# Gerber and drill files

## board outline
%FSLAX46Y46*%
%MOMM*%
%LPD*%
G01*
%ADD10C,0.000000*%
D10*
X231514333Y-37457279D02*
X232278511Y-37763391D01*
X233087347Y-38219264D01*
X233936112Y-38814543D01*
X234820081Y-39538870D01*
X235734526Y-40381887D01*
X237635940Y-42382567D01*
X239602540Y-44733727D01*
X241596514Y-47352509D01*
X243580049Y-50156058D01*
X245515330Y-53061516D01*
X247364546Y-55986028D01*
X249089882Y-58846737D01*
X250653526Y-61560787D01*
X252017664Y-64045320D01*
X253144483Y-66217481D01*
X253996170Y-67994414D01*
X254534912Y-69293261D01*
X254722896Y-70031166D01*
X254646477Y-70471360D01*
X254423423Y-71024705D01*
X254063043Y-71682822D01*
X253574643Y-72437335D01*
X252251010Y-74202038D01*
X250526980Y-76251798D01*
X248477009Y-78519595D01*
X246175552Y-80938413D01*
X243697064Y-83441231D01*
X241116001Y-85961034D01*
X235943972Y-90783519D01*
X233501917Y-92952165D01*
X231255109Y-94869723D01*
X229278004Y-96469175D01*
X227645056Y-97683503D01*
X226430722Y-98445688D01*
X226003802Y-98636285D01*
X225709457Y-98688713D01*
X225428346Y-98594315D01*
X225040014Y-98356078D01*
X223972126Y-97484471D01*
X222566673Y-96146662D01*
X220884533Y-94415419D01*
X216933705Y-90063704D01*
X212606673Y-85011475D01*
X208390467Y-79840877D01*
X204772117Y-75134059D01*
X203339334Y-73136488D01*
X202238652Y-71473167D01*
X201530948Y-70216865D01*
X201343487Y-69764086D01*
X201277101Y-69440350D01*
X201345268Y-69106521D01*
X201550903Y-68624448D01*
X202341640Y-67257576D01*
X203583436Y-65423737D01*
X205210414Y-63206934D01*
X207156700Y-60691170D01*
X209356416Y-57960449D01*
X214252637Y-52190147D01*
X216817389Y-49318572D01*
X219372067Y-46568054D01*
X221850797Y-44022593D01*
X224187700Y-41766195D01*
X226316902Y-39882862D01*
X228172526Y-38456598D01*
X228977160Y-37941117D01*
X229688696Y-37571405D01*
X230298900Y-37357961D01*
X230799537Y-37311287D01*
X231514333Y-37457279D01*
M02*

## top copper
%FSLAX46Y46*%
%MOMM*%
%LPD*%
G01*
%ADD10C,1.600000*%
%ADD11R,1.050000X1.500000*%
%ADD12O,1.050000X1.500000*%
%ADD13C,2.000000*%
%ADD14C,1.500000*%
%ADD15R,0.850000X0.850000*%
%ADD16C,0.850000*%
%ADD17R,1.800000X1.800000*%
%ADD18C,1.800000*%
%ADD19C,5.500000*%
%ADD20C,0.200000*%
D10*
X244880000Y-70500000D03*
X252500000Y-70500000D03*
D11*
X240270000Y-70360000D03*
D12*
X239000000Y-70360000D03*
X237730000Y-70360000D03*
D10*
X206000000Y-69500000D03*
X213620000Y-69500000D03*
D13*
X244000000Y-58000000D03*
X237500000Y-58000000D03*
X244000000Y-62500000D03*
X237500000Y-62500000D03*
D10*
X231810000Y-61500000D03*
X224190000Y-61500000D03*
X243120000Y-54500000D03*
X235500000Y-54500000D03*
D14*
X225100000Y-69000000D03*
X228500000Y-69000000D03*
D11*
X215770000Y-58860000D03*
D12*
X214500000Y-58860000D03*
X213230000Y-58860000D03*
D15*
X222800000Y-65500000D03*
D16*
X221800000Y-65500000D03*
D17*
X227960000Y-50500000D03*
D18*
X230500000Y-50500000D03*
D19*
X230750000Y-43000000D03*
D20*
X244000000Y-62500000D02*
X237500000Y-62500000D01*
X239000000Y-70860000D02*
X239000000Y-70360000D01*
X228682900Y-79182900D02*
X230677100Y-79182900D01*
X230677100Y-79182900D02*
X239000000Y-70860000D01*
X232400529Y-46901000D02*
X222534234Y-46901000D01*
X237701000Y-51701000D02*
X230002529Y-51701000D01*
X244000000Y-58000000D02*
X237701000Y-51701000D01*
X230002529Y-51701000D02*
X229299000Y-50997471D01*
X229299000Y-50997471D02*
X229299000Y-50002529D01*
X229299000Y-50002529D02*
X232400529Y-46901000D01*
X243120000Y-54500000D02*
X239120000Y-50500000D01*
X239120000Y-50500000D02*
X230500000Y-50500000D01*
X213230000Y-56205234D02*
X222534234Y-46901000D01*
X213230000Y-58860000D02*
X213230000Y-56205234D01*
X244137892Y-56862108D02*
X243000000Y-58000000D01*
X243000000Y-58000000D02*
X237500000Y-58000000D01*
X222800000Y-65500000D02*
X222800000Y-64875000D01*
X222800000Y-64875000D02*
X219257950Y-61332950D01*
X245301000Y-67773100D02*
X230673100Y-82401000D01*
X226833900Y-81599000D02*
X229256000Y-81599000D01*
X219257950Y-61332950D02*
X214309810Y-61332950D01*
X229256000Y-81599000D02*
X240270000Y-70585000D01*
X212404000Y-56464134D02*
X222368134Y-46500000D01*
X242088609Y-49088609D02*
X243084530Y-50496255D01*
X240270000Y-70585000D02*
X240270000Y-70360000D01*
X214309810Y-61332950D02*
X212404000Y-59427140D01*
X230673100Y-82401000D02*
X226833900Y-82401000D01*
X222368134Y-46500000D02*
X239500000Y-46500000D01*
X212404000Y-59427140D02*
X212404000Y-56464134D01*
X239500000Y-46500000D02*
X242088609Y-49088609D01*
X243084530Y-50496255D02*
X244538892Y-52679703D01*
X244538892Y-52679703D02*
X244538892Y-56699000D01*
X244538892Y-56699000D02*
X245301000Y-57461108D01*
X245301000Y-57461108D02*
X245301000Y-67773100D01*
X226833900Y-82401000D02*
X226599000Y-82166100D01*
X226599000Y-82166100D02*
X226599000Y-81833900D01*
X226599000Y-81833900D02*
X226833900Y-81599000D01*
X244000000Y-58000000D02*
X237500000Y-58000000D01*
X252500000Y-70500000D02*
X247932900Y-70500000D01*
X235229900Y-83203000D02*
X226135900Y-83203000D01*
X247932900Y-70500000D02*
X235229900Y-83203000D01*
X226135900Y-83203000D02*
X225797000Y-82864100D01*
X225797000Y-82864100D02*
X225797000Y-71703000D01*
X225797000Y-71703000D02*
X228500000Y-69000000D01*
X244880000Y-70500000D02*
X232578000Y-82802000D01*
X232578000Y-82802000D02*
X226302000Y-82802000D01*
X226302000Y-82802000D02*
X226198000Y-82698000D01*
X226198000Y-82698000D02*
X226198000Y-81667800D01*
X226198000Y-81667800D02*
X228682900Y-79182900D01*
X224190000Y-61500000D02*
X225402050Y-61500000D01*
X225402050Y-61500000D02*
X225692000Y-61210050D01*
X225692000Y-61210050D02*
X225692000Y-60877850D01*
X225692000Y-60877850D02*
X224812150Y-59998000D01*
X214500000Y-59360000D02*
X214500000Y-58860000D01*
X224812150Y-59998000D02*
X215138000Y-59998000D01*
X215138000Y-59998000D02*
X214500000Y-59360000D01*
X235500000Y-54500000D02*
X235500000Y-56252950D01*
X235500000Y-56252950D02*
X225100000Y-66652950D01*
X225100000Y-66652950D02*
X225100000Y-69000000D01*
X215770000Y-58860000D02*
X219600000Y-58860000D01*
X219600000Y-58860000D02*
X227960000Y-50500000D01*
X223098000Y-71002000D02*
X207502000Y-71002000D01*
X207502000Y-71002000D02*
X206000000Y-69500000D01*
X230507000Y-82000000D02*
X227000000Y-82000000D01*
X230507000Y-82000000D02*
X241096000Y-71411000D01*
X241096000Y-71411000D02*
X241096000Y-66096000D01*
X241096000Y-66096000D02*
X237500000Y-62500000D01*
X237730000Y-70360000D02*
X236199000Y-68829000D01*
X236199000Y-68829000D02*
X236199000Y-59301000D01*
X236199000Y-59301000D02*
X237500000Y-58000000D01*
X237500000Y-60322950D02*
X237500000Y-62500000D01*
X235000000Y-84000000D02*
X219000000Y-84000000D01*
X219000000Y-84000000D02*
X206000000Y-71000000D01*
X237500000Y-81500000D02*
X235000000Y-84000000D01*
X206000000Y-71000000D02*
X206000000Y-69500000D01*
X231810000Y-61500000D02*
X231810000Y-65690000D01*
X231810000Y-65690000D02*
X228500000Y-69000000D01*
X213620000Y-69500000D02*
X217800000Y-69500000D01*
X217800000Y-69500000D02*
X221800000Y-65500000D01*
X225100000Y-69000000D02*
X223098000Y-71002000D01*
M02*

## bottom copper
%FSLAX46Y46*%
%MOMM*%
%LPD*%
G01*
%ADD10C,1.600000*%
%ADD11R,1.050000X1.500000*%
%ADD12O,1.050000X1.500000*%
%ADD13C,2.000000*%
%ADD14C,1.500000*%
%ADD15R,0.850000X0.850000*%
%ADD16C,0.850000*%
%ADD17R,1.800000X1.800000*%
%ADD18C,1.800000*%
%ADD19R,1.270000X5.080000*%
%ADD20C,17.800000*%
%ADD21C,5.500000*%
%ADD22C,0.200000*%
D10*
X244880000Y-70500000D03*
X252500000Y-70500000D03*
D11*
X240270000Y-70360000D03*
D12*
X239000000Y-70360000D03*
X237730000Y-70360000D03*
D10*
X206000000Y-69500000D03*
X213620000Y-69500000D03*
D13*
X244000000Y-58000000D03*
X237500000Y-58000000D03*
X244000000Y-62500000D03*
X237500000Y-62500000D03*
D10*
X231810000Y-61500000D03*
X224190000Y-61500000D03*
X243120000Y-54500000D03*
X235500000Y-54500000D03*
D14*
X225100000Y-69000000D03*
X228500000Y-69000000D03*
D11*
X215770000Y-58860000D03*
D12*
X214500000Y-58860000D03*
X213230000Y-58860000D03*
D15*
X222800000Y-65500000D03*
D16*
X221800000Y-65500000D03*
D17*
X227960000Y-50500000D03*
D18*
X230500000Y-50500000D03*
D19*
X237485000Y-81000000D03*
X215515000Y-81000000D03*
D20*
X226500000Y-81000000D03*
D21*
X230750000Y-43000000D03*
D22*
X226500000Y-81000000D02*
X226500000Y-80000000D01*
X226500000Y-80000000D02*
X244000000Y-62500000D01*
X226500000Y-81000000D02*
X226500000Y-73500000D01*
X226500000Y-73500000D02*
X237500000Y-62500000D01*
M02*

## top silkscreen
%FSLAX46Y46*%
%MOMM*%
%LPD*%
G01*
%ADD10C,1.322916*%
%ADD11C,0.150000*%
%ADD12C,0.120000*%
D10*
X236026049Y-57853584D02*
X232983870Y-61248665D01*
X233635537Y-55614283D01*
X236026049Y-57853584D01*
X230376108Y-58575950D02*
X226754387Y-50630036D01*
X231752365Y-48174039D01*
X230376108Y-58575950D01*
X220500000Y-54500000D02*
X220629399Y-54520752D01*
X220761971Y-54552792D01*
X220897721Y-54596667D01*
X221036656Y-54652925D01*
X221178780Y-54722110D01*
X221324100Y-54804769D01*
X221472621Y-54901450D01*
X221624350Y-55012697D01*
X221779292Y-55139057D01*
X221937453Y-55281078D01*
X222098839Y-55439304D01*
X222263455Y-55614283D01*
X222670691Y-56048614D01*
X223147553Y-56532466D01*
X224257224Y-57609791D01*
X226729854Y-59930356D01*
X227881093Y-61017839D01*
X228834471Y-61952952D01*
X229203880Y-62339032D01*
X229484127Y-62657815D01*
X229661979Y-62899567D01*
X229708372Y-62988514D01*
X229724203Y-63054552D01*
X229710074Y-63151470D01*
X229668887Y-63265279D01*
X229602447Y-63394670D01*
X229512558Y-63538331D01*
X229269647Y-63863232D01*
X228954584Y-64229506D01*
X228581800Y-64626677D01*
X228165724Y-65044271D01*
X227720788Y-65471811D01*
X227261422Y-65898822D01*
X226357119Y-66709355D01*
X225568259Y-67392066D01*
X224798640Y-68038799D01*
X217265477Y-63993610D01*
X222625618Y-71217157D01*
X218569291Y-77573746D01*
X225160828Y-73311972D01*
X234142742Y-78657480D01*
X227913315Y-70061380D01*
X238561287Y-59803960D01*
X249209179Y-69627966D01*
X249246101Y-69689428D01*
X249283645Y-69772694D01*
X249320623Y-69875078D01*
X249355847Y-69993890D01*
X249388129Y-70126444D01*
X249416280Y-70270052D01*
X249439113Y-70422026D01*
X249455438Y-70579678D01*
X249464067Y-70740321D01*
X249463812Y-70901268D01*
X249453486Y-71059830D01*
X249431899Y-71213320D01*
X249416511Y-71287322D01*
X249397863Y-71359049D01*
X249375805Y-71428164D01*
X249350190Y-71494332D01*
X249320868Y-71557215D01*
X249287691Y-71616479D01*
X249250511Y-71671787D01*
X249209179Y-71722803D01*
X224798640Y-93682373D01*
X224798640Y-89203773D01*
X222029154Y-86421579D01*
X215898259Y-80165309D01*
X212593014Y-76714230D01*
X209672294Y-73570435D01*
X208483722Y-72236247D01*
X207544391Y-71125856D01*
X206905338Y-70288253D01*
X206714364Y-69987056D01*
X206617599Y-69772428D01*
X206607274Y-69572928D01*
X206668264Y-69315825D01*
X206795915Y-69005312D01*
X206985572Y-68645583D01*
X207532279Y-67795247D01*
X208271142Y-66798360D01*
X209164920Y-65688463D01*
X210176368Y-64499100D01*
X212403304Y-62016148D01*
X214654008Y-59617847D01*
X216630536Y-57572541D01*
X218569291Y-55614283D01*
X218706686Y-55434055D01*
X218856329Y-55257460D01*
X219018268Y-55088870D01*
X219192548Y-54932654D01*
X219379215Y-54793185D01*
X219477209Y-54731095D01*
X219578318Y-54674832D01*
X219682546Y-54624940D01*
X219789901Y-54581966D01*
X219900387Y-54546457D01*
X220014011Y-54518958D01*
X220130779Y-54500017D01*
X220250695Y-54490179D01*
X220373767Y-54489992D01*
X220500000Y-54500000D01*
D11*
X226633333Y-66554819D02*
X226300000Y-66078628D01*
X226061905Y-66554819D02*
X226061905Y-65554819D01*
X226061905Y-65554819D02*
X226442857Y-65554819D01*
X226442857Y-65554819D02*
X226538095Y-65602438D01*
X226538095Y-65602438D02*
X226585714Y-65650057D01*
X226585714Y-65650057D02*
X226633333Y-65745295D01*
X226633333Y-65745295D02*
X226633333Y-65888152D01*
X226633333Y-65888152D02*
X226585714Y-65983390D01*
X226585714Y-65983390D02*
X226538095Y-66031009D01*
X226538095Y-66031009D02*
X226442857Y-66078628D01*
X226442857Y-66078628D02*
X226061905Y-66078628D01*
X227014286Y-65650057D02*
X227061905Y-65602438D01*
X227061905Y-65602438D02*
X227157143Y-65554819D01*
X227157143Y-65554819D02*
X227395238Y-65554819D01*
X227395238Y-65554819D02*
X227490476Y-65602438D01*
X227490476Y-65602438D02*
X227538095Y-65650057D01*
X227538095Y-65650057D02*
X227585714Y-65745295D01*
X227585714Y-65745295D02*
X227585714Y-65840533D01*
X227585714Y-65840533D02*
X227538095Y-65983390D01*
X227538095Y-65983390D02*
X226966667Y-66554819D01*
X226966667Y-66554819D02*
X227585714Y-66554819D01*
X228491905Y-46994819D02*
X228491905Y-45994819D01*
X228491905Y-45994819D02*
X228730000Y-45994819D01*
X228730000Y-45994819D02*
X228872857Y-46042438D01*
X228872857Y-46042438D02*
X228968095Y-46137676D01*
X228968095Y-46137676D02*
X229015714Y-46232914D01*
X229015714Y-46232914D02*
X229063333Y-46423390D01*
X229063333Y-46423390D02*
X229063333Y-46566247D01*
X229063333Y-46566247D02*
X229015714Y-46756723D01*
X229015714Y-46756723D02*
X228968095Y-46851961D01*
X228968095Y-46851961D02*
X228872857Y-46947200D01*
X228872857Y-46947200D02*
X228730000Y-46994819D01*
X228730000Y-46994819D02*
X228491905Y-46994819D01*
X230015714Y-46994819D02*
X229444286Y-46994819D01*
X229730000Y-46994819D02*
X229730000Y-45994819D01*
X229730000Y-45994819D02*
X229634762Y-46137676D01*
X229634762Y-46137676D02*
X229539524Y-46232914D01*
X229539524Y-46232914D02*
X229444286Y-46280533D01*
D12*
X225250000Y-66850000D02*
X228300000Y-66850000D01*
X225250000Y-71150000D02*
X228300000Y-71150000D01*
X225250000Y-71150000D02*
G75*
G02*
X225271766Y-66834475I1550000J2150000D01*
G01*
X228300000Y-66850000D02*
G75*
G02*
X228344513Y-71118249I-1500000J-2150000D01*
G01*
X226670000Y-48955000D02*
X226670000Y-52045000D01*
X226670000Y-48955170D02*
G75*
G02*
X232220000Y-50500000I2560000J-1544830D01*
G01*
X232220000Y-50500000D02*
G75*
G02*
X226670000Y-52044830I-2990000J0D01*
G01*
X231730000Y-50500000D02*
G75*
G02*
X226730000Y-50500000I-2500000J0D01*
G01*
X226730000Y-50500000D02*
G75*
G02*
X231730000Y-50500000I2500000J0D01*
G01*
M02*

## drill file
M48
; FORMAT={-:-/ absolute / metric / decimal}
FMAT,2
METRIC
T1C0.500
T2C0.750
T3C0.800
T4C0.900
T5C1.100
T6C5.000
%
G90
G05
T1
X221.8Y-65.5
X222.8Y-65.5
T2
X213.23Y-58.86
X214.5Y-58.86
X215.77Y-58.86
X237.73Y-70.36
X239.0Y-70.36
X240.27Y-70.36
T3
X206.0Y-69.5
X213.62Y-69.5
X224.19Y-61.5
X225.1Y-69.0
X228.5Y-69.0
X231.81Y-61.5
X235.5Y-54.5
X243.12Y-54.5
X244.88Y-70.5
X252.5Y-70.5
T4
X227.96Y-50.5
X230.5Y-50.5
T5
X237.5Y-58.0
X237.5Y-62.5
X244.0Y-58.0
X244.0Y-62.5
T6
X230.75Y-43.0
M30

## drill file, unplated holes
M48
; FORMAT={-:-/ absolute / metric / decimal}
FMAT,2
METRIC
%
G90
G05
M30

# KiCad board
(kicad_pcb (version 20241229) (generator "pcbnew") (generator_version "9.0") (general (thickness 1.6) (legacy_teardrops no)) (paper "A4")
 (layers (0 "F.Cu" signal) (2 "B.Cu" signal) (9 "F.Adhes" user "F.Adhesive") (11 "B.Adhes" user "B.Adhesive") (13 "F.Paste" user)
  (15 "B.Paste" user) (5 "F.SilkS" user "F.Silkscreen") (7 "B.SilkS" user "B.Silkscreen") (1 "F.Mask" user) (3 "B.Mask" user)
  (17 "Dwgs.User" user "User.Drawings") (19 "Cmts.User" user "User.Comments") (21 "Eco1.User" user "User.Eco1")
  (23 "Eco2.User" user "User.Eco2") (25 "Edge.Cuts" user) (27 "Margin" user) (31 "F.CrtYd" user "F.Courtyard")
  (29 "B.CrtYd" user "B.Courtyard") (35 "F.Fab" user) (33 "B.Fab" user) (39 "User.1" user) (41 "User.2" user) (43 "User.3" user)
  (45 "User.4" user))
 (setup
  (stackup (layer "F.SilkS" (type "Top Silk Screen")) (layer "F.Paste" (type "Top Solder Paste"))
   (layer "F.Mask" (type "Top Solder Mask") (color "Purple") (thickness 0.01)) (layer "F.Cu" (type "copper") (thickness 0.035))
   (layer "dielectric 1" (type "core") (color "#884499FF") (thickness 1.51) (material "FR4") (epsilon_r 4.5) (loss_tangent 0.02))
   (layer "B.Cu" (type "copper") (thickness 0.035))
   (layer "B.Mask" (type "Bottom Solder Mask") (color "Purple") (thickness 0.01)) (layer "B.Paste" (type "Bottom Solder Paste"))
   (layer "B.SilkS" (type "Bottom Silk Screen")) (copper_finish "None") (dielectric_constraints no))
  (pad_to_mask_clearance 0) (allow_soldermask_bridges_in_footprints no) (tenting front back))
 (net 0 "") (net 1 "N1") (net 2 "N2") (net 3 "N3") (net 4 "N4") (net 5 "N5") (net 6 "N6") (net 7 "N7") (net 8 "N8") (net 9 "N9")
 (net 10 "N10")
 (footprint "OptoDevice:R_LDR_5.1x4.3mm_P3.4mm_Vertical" (layer "F.Cu") (at 225.1 69)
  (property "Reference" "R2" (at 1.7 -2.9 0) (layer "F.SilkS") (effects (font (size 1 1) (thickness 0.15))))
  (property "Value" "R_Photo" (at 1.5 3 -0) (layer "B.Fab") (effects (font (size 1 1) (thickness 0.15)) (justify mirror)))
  (fp_line (start 0.15 -2.15) (end 3.2 -2.15) (stroke (width 0.12) (type solid)) (layer "F.SilkS"))
  (fp_line (start 0.15 2.15) (end 3.2 2.15) (stroke (width 0.12) (type solid)) (layer "F.SilkS"))
  (fp_arc (start 0.15 2.15) (mid -0.950438 -0.013368) (end 0.171766 -2.165525) (stroke (width 0.12) (type solid)) (layer "F.SilkS"))
  (fp_arc (start 3.2 -2.15) (mid 4.321403 -0.027338) (end 3.244513 2.118249) (stroke (width 0.12) (type solid)) (layer "F.SilkS"))
  (pad "1" thru_hole circle (at 0 0) (size 1.5 1.5) (drill 0.8) (layers "*.Cu" "*.Mask") (remove_unused_layers no) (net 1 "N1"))
  (pad "2" thru_hole circle (at 3.4 0) (size 1.5 1.5) (drill 0.8) (layers "*.Cu" "*.Mask") (remove_unused_layers no) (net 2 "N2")))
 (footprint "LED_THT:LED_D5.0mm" (layer "F.Cu") (at 227.96 50.5)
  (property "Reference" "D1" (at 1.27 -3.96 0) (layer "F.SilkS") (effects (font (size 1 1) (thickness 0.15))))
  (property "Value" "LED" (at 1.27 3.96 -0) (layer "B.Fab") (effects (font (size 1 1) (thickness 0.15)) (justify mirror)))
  (fp_line (start -1.29 -1.545) (end -1.29 1.545) (stroke (width 0.12) (type solid)) (layer "F.SilkS"))
  (fp_arc (start -1.29 -1.54483) (mid 2.071779 -2.880495) (end 4.26 0) (stroke (width 0.12) (type solid)) (layer "F.SilkS"))
  (fp_arc (start 4.26 0) (mid 2.071779 2.880495) (end -1.29 1.54483) (stroke (width 0.12) (type solid)) (layer "F.SilkS"))
  (fp_circle (center 1.27 0) (end 3.77 0) (stroke (width 0.12) (type solid)) (fill no) (layer "F.SilkS"))
  (pad "1" thru_hole rect (at 0 0) (size 1.8 1.8) (drill 0.9) (layers "*.Cu" "*.Mask") (remove_unused_layers no) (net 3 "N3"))
  (pad "2" thru_hole circle (at 2.54 0) (size 1.8 1.8) (drill 0.9) (layers "*.Cu" "*.Mask") (remove_unused_layers no) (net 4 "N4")))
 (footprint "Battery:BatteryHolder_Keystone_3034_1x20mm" (layer "B.Cu") (at 226.5 81 180)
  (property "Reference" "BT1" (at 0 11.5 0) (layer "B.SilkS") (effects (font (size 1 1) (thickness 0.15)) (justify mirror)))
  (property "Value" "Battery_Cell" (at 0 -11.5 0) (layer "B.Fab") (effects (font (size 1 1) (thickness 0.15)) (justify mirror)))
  (pad "1" smd rect (at -10.985 0 180) (size 1.27 5.08) (layers "B.Cu" "B.Mask" "B.Paste") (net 1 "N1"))
  (pad "1" smd rect (at 10.985 0 180) (size 1.27 5.08) (layers "B.Cu" "B.Mask" "B.Paste") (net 1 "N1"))
  (pad "2" smd circle (at 0 0 180) (size 17.8 17.8) (layers "B.Cu" "B.Mask") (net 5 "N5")))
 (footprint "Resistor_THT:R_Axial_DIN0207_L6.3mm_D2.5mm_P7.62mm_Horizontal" (layer "B.Cu") (at 231.81 61.5 180)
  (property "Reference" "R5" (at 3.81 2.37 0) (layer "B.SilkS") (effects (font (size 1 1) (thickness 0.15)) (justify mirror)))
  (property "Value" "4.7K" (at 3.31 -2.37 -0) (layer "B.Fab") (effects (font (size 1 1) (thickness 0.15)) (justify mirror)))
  (pad "1" thru_hole circle (at 0 0 180) (size 1.6 1.6) (drill 0.8) (layers "*.Cu" "*.Mask") (remove_unused_layers no) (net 2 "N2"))
  (pad "2" thru_hole circle (at 7.62 0 180) (size 1.6 1.6) (drill 0.8) (layers "*.Cu" "*.Mask") (remove_unused_layers no) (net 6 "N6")))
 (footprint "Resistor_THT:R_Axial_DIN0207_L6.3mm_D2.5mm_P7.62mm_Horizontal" (layer "B.Cu") (at 243.12 54.5 180)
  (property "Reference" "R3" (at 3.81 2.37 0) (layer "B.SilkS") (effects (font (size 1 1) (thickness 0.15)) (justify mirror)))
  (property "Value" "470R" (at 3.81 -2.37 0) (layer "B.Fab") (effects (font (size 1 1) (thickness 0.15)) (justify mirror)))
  (pad "1" thru_hole circle (at 0 0 180) (size 1.6 1.6) (drill 0.8) (layers "*.Cu" "*.Mask") (remove_unused_layers no) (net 4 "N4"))
  (pad "2" thru_hole circle (at 7.62 0 180) (size 1.6 1.6) (drill 0.8) (layers "*.Cu" "*.Mask") (remove_unused_layers no) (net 1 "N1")))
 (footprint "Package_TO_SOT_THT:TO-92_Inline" (layer "B.Cu") (at 240.27 70.36 180)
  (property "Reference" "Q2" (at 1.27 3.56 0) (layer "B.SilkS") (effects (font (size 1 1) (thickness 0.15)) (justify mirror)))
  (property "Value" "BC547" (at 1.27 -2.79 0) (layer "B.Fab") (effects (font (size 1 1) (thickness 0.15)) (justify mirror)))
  (pad "1" thru_hole rect (at 0 0 180) (size 1.05 1.5) (drill 0.75) (layers "*.Cu" "*.Mask") (remove_unused_layers no) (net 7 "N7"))
  (pad "2" thru_hole oval (at 1.27 0 180) (size 1.05 1.5) (drill 0.75) (layers "*.Cu" "*.Mask") (remove_unused_layers no) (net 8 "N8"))
  (pad "3" thru_hole oval (at 2.54 0 180) (size 1.05 1.5) (drill 0.75) (layers "*.Cu" "*.Mask") (remove_unused_layers no) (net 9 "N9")))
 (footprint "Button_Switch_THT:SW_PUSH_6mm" (layer "B.Cu") (at 244 58 180)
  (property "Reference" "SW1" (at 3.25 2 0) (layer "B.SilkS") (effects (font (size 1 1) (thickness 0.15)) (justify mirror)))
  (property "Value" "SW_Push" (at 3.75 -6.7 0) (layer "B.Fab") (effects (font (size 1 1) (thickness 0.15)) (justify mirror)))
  (pad "1" thru_hole circle (at 0 0 90) (size 2 2) (drill 1.1) (layers "*.Cu" "*.Mask") (remove_unused_layers no) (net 9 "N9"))
  (pad "1" thru_hole circle (at 6.5 0 90) (size 2 2) (drill 1.1) (layers "*.Cu" "*.Mask") (remove_unused_layers no) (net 9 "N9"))
  (pad "2" thru_hole circle (at 0 -4.5 90) (size 2 2) (drill 1.1) (layers "*.Cu" "*.Mask") (remove_unused_layers no) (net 5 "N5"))
  (pad "2" thru_hole circle (at 6.5 -4.5 90) (size 2 2) (drill 1.1) (layers "*.Cu" "*.Mask") (remove_unused_layers no) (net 5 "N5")))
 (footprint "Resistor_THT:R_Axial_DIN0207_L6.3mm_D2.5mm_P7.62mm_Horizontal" (layer "B.Cu") (at 213.62 69.5 180)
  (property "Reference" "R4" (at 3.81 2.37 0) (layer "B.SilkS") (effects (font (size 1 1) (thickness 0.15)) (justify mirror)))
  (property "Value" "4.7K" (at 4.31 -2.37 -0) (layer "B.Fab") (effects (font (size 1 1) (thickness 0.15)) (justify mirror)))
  (pad "1" thru_hole circle (at 0 0 180) (size 1.6 1.6) (drill 0.8) (layers "*.Cu" "*.Mask") (remove_unused_layers no) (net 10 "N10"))
  (pad "2" thru_hole circle (at 7.62 0 180) (size 1.6 1.6) (drill 0.8) (layers "*.Cu" "*.Mask") (remove_unused_layers no) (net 1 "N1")))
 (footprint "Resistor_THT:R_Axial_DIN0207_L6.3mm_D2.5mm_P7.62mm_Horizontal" (layer "B.Cu") (at 252.5 70.5 180)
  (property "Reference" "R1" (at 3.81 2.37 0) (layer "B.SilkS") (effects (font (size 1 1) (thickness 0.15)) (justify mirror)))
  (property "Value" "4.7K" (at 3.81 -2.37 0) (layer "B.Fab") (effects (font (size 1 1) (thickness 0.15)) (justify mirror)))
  (pad "1" thru_hole circle (at 0 0 180) (size 1.6 1.6) (drill 0.8) (layers "*.Cu" "*.Mask") (remove_unused_layers no) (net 2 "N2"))
  (pad "2" thru_hole circle (at 7.62 0 180) (size 1.6 1.6) (drill 0.8) (layers "*.Cu" "*.Mask") (remove_unused_layers no) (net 8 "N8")))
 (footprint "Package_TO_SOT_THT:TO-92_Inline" (layer "B.Cu") (at 215.77 58.86 180)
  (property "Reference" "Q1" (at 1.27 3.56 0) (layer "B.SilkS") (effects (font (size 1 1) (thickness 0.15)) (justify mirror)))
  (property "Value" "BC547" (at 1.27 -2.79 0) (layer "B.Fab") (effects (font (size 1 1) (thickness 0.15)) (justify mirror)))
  (pad "1" thru_hole rect (at 0 0 180) (size 1.05 1.5) (drill 0.75) (layers "*.Cu" "*.Mask") (remove_unused_layers no) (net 3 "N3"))
  (pad "2" thru_hole oval (at 1.27 0 180) (size 1.05 1.5) (drill 0.75) (layers "*.Cu" "*.Mask") (remove_unused_layers no) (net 6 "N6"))
  (pad "3" thru_hole oval (at 2.54 0 180) (size 1.05 1.5) (drill 0.75) (layers "*.Cu" "*.Mask") (remove_unused_layers no) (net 9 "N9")))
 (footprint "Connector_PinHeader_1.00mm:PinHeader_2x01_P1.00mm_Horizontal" (layer "B.Cu") (at 222.8 65.5 180)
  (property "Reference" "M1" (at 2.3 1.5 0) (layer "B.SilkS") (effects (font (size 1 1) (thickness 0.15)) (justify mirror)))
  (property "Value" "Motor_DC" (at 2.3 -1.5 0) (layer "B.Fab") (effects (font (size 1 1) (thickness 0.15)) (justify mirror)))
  (pad "1" thru_hole rect (at 0 0 180) (size 0.85 0.85) (drill 0.5) (layers "*.Cu" "*.Mask") (remove_unused_layers no) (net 7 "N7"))
  (pad "2" thru_hole circle (at 1 0 180) (size 0.85 0.85) (drill 0.5) (layers "*.Cu" "*.Mask") (remove_unused_layers no) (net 10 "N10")))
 (gr_poly
  (pts (xy 236.026049 57.853584) (xy 232.98387 61.248665) (xy 233.635537 55.614283))
  (stroke (width 1.322916) (type solid) (color 255 255 255 1)) (fill no) (layer "F.SilkS"))
 (gr_poly
  (pts (xy 230.376108 58.57595) (xy 226.754387 50.630036) (xy 231.752365 48.174039))
  (stroke (width 1.322916) (type solid) (color 255 255 255 1)) (fill no) (layer "F.SilkS"))
 (gr_poly
  (pts (xy 220.5 54.5) (xy 220.629399 54.520752) (xy 220.761971 54.552792) (xy 220.897721 54.596667) (xy 221.036656 54.652925)
   (xy 221.17878 54.72211) (xy 221.3241 54.804769) (xy 221.472621 54.90145) (xy 221.62435 55.012697) (xy 221.779292 55.139057)
   (xy 221.937453 55.281078) (xy 222.098839 55.439304) (xy 222.263455 55.614283) (xy 222.670691 56.048614) (xy 223.147553 56.532466)
   (xy 224.257224 57.609791) (xy 226.729854 59.930356) (xy 227.881093 61.017839) (xy 228.834471 61.952952) (xy 229.20388 62.339032)
   (xy 229.484127 62.657815) (xy 229.661979 62.899567) (xy 229.708372 62.988514) (xy 229.724203 63.054552) (xy 229.710074 63.15147)
   (xy 229.668887 63.265279) (xy 229.602447 63.39467) (xy 229.512558 63.538331) (xy 229.269647 63.863232) (xy 228.954584 64.229506)
   (xy 228.5818 64.626677) (xy 228.165724 65.044271) (xy 227.720788 65.471811) (xy 227.261422 65.898822) (xy 226.357119 66.709355)
   (xy 225.568259 67.392066) (xy 224.79864 68.038799) (xy 217.265477 63.99361) (xy 222.625618 71.217157) (xy 218.569291 77.573746)
   (xy 225.160828 73.311972) (xy 234.142742 78.65748) (xy 227.913315 70.06138) (xy 238.561287 59.80396) (xy 249.209179 69.627966)
   (xy 249.246101 69.689428) (xy 249.283645 69.772694) (xy 249.320623 69.875078) (xy 249.355847 69.99389) (xy 249.388129 70.126444)
   (xy 249.41628 70.270052) (xy 249.439113 70.422026) (xy 249.455438 70.579678) (xy 249.464067 70.740321) (xy 249.463812 70.901268)
   (xy 249.453486 71.05983) (xy 249.431899 71.21332) (xy 249.416511 71.287322) (xy 249.397863 71.359049) (xy 249.375805 71.428164)
   (xy 249.35019 71.494332) (xy 249.320868 71.557215) (xy 249.287691 71.616479) (xy 249.250511 71.671787) (xy 249.209179 71.722803)
   (xy 224.79864 93.682373) (xy 224.79864 89.203773) (xy 222.029154 86.421579) (xy 215.898259 80.165309) (xy 212.593014 76.71423)
   (xy 209.672294 73.570435) (xy 208.483722 72.236247) (xy 207.544391 71.125856) (xy 206.905338 70.288253) (xy 206.714364 69.987056)
   (xy 206.617599 69.772428) (xy 206.607274 69.572928) (xy 206.668264 69.315825) (xy 206.795915 69.005312) (xy 206.985572 68.645583)
   (xy 207.532279 67.795247) (xy 208.271142 66.79836) (xy 209.16492 65.688463) (xy 210.176368 64.4991) (xy 212.403304 62.016148)
   (xy 214.654008 59.617847) (xy 216.630536 57.572541) (xy 218.569291 55.614283) (xy 218.706686 55.434055) (xy 218.856329 55.25746)
   (xy 219.018268 55.08887) (xy 219.192548 54.932654) (xy 219.379215 54.793185) (xy 219.477209 54.731095) (xy 219.578318 54.674832)
   (xy 219.682546 54.62494) (xy 219.789901 54.581966) (xy 219.900387 54.546457) (xy 220.014011 54.518958) (xy 220.130779 54.500017)
   (xy 220.250695 54.490179) (xy 220.373767 54.489992))
  (stroke (width 1.322916) (type solid) (color 255 255 255 1)) (fill no) (layer "F.SilkS"))
 (gr_poly
  (pts (xy 231.514333 37.457279) (xy 232.278511 37.763391) (xy 233.087347 38.219264) (xy 233.936112 38.814543) (xy 234.820081 39.53887)
   (xy 235.734526 40.381887) (xy 237.63594 42.382567) (xy 239.60254 44.733727) (xy 241.596514 47.352509) (xy 243.580049 50.156058)
   (xy 245.51533 53.061516) (xy 247.364546 55.986028) (xy 249.089882 58.846737) (xy 250.653526 61.560787) (xy 252.017664 64.04532)
   (xy 253.144483 66.217481) (xy 253.99617 67.994414) (xy 254.534912 69.293261) (xy 254.722896 70.031166) (xy 254.646477 70.47136)
   (xy 254.423423 71.024705) (xy 254.063043 71.682822) (xy 253.574643 72.437335) (xy 252.25101 74.202038) (xy 250.52698 76.251798)
   (xy 248.477009 78.519595) (xy 246.175552 80.938413) (xy 243.697064 83.441231) (xy 241.116001 85.961034) (xy 235.943972 90.783519)
   (xy 233.501917 92.952165) (xy 231.255109 94.869723) (xy 229.278004 96.469175) (xy 227.645056 97.683503) (xy 226.430722 98.445688)
   (xy 226.003802 98.636285) (xy 225.709457 98.688713) (xy 225.428346 98.594315) (xy 225.040014 98.356078) (xy 223.972126 97.484471)
   (xy 222.566673 96.146662) (xy 220.884533 94.415419) (xy 216.933705 90.063704) (xy 212.606673 85.011475) (xy 208.390467 79.840877)
   (xy 204.772117 75.134059) (xy 203.339334 73.136488) (xy 202.238652 71.473167) (xy 201.530948 70.216865) (xy 201.343487 69.764086)
   (xy 201.277101 69.44035) (xy 201.345268 69.106521) (xy 201.550903 68.624448) (xy 202.34164 67.257576) (xy 203.583436 65.423737)
   (xy 205.210414 63.206934) (xy 207.1567 60.69117) (xy 209.356416 57.960449) (xy 214.252637 52.190147) (xy 216.817389 49.318572)
   (xy 219.372067 46.568054) (xy 221.850797 44.022593) (xy 224.1877 41.766195) (xy 226.316902 39.882862) (xy 228.172526 38.456598)
   (xy 228.97716 37.941117) (xy 229.688696 37.571405) (xy 230.2989 37.357961) (xy 230.799537 37.311287))
  (stroke (width 0) (type solid) (color 255 255 255 1)) (fill no) (layer "Edge.Cuts"))
 (via (at 230.75 43) (size 5.5) (drill 5) (layers "F.Cu" "B.Cu") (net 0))
 (segment (start 235.5 54.5) (end 235.5 56.25295) (width 0.2) (layer "F.Cu") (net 1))
 (segment (start 207.502 71.002) (end 206 69.5) (width 0.2) (layer "F.Cu") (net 1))
 (segment (start 225.1 69) (end 223.098 71.002) (width 0.2) (layer "F.Cu") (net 1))
 (segment (start 206 71) (end 206 69.5) (width 0.2) (layer "F.Cu") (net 1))
 (segment (start 235 84) (end 219 84) (width 0.2) (layer "F.Cu") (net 1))
 (segment (start 223.098 71.002) (end 207.502 71.002) (width 0.2) (layer "F.Cu") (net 1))
 (segment (start 219 84) (end 206 71) (width 0.2) (layer "F.Cu") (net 1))
 (segment (start 225.1 66.65295) (end 225.1 69) (width 0.2) (layer "F.Cu") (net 1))
 (segment (start 235.5 56.25295) (end 225.1 66.65295) (width 0.2) (layer "F.Cu") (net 1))
 (segment (start 237.5 81.5) (end 235 84) (width 0.2) (layer "F.Cu") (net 1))
 (segment (start 244 62.5) (end 237.5 62.5) (width 0.2) (layer "F.Cu") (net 5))
 (segment (start 230.507 82) (end 227 82) (width 0.2) (layer "F.Cu") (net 5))
 (segment (start 241.096 71.411) (end 241.096 66.096) (width 0.2) (layer "F.Cu") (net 5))
 (segment (start 241.096 66.096) (end 237.5 62.5) (width 0.2) (layer "F.Cu") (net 5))
 (segment (start 237.5 60.32295) (end 237.5 62.5) (width 0.2) (layer "F.Cu") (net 5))
 (segment (start 230.507 82) (end 241.096 71.411) (width 0.2) (layer "F.Cu") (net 5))
 (segment (start 226.5 80) (end 244 62.5) (width 0.2) (layer "B.Cu") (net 5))
 (segment (start 226.5 73.5) (end 237.5 62.5) (width 0.2) (layer "B.Cu") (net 5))
 (segment (start 226.5 81) (end 226.5 80) (width 0.2) (layer "B.Cu") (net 5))
 (segment (start 226.5 81) (end 226.5 73.5) (width 0.2) (layer "B.Cu") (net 5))
 (segment (start 239.12 50.5) (end 230.5 50.5) (width 0.2) (layer "F.Cu") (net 4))
 (segment (start 243.12 54.5) (end 239.12 50.5) (width 0.2) (layer "F.Cu") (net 4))
 (segment (start 215.77 58.86) (end 219.6 58.86) (width 0.2) (layer "F.Cu") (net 3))
 (segment (start 219.6 58.86) (end 227.96 50.5) (width 0.2) (layer "F.Cu") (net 3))
 (segment (start 244 58) (end 237.5 58) (width 0.2) (layer "F.Cu") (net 9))
 (segment (start 236.199 59.301) (end 237.5 58) (width 0.2) (layer "F.Cu") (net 9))
 (segment (start 243 58) (end 237.5 58) (width 0.2) (layer "F.Cu") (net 9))
 (segment (start 213.23 58.86) (end 213.23 56.205234) (width 0.2) (layer "F.Cu") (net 9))
 (segment (start 237.701 51.701) (end 230.002529 51.701) (width 0.2) (layer "F.Cu") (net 9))
 (segment (start 237.73 70.36) (end 236.199 68.829) (width 0.2) (layer "F.Cu") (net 9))
 (segment (start 229.299 50.002529) (end 232.400529 46.901) (width 0.2) (layer "F.Cu") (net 9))
 (segment (start 244 58) (end 237.701 51.701) (width 0.2) (layer "F.Cu") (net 9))
 (segment (start 213.23 56.205234) (end 222.534234 46.901) (width 0.2) (layer "F.Cu") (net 9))
 (segment (start 236.199 68.829) (end 236.199 59.301) (width 0.2) (layer "F.Cu") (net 9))
 (segment (start 244.137892 56.862108) (end 243 58) (width 0.2) (layer "F.Cu") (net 9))
 (segment (start 229.299 50.997471) (end 229.299 50.002529) (width 0.2) (layer "F.Cu") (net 9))
 (segment (start 230.002529 51.701) (end 229.299 50.997471) (width 0.2) (layer "F.Cu") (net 9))
 (segment (start 232.400529 46.901) (end 222.534234 46.901) (width 0.2) (layer "F.Cu") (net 9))
 (segment (start 225.692 60.87785) (end 224.81215 59.998) (width 0.2) (layer "F.Cu") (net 6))
 (segment (start 224.81215 59.998) (end 215.138 59.998) (width 0.2) (layer "F.Cu") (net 6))
 (segment (start 225.40205 61.5) (end 225.692 61.21005) (width 0.2) (layer "F.Cu") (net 6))
 (segment (start 225.692 61.21005) (end 225.692 60.87785) (width 0.2) (layer "F.Cu") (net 6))
 (segment (start 214.5 59.36) (end 214.5 58.86) (width 0.2) (layer "F.Cu") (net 6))
 (segment (start 224.19 61.5) (end 225.40205 61.5) (width 0.2) (layer "F.Cu") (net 6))
 (segment (start 215.138 59.998) (end 214.5 59.36) (width 0.2) (layer "F.Cu") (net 6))
 (segment (start 222.368134 46.5) (end 239.5 46.5) (width 0.2) (layer "F.Cu") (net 7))
 (segment (start 222.8 64.875) (end 219.25795 61.33295) (width 0.2) (layer "F.Cu") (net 7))
 (segment (start 243.08453 50.496255) (end 244.538892 52.679703) (width 0.2) (layer "F.Cu") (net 7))
 (segment (start 212.404 59.42714) (end 212.404 56.464134) (width 0.2) (layer "F.Cu") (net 7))
 (segment (start 244.538892 56.699) (end 245.301 57.461108) (width 0.2) (layer "F.Cu") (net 7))
 (segment (start 226.599 82.1661) (end 226.599 81.8339) (width 0.2) (layer "F.Cu") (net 7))
 (segment (start 212.404 56.464134) (end 222.368134 46.5) (width 0.2) (layer "F.Cu") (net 7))
 (segment (start 245.301 67.7731) (end 230.6731 82.401) (width 0.2) (layer "F.Cu") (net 7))
 (segment (start 242.088609 49.088609) (end 243.08453 50.496255) (width 0.2) (layer "F.Cu") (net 7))
 (segment (start 226.8339 82.401) (end 226.599 82.1661) (width 0.2) (layer "F.Cu") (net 7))
 (segment (start 226.8339 81.599) (end 229.256 81.599) (width 0.2) (layer "F.Cu") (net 7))
 (segment (start 245.301 57.461108) (end 245.301 67.7731) (width 0.2) (layer "F.Cu") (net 7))
 (segment (start 219.25795 61.33295) (end 214.30981 61.33295) (width 0.2) (layer "F.Cu") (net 7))
 (segment (start 214.30981 61.33295) (end 212.404 59.42714) (width 0.2) (layer "F.Cu") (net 7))
 (segment (start 222.8 65.5) (end 222.8 64.875) (width 0.2) (layer "F.Cu") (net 7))
 (segment (start 239.5 46.5) (end 242.088609 49.088609) (width 0.2) (layer "F.Cu") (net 7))
 (segment (start 244.538892 52.679703) (end 244.538892 56.699) (width 0.2) (layer "F.Cu") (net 7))
 (segment (start 226.599 81.8339) (end 226.8339 81.599) (width 0.2) (layer "F.Cu") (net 7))
 (segment (start 240.27 70.585) (end 240.27 70.36) (width 0.2) (layer "F.Cu") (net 7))
 (segment (start 230.6731 82.401) (end 226.8339 82.401) (width 0.2) (layer "F.Cu") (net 7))
 (segment (start 229.256 81.599) (end 240.27 70.585) (width 0.2) (layer "F.Cu") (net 7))
 (segment (start 217.8 69.5) (end 221.8 65.5) (width 0.2) (layer "F.Cu") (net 10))
 (segment (start 213.62 69.5) (end 217.8 69.5) (width 0.2) (layer "F.Cu") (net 10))
 (segment (start 228.6829 79.1829) (end 230.6771 79.1829) (width 0.2) (layer "F.Cu") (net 8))
 (segment (start 226.198 82.698) (end 226.198 81.6678) (width 0.2) (layer "F.Cu") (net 8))
 (segment (start 239 70.86) (end 239 70.36) (width 0.2) (layer "F.Cu") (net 8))
 (segment (start 230.6771 79.1829) (end 239 70.86) (width 0.2) (layer "F.Cu") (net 8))
 (segment (start 232.578 82.802) (end 226.302 82.802) (width 0.2) (layer "F.Cu") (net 8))
 (segment (start 226.198 81.6678) (end 228.6829 79.1829) (width 0.2) (layer "F.Cu") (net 8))
 (segment (start 244.88 70.5) (end 232.578 82.802) (width 0.2) (layer "F.Cu") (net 8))
 (segment (start 226.302 82.802) (end 226.198 82.698) (width 0.2) (layer "F.Cu") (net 8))
 (segment (start 225.797 82.8641) (end 225.797 71.703) (width 0.2) (layer "F.Cu") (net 2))
 (segment (start 231.81 65.69) (end 228.5 69) (width 0.2) (layer "F.Cu") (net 2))
 (segment (start 247.9329 70.5) (end 235.2299 83.203) (width 0.2) (layer "F.Cu") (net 2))
 (segment (start 252.5 70.5) (end 247.9329 70.5) (width 0.2) (layer "F.Cu") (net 2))
 (segment (start 226.1359 83.203) (end 225.797 82.8641) (width 0.2) (layer "F.Cu") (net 2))
 (segment (start 225.797 71.703) (end 228.5 69) (width 0.2) (layer "F.Cu") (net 2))
 (segment (start 235.2299 83.203) (end 226.1359 83.203) (width 0.2) (layer "F.Cu") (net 2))
 (segment (start 231.81 61.5) (end 231.81 65.69) (width 0.2) (layer "F.Cu") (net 2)))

